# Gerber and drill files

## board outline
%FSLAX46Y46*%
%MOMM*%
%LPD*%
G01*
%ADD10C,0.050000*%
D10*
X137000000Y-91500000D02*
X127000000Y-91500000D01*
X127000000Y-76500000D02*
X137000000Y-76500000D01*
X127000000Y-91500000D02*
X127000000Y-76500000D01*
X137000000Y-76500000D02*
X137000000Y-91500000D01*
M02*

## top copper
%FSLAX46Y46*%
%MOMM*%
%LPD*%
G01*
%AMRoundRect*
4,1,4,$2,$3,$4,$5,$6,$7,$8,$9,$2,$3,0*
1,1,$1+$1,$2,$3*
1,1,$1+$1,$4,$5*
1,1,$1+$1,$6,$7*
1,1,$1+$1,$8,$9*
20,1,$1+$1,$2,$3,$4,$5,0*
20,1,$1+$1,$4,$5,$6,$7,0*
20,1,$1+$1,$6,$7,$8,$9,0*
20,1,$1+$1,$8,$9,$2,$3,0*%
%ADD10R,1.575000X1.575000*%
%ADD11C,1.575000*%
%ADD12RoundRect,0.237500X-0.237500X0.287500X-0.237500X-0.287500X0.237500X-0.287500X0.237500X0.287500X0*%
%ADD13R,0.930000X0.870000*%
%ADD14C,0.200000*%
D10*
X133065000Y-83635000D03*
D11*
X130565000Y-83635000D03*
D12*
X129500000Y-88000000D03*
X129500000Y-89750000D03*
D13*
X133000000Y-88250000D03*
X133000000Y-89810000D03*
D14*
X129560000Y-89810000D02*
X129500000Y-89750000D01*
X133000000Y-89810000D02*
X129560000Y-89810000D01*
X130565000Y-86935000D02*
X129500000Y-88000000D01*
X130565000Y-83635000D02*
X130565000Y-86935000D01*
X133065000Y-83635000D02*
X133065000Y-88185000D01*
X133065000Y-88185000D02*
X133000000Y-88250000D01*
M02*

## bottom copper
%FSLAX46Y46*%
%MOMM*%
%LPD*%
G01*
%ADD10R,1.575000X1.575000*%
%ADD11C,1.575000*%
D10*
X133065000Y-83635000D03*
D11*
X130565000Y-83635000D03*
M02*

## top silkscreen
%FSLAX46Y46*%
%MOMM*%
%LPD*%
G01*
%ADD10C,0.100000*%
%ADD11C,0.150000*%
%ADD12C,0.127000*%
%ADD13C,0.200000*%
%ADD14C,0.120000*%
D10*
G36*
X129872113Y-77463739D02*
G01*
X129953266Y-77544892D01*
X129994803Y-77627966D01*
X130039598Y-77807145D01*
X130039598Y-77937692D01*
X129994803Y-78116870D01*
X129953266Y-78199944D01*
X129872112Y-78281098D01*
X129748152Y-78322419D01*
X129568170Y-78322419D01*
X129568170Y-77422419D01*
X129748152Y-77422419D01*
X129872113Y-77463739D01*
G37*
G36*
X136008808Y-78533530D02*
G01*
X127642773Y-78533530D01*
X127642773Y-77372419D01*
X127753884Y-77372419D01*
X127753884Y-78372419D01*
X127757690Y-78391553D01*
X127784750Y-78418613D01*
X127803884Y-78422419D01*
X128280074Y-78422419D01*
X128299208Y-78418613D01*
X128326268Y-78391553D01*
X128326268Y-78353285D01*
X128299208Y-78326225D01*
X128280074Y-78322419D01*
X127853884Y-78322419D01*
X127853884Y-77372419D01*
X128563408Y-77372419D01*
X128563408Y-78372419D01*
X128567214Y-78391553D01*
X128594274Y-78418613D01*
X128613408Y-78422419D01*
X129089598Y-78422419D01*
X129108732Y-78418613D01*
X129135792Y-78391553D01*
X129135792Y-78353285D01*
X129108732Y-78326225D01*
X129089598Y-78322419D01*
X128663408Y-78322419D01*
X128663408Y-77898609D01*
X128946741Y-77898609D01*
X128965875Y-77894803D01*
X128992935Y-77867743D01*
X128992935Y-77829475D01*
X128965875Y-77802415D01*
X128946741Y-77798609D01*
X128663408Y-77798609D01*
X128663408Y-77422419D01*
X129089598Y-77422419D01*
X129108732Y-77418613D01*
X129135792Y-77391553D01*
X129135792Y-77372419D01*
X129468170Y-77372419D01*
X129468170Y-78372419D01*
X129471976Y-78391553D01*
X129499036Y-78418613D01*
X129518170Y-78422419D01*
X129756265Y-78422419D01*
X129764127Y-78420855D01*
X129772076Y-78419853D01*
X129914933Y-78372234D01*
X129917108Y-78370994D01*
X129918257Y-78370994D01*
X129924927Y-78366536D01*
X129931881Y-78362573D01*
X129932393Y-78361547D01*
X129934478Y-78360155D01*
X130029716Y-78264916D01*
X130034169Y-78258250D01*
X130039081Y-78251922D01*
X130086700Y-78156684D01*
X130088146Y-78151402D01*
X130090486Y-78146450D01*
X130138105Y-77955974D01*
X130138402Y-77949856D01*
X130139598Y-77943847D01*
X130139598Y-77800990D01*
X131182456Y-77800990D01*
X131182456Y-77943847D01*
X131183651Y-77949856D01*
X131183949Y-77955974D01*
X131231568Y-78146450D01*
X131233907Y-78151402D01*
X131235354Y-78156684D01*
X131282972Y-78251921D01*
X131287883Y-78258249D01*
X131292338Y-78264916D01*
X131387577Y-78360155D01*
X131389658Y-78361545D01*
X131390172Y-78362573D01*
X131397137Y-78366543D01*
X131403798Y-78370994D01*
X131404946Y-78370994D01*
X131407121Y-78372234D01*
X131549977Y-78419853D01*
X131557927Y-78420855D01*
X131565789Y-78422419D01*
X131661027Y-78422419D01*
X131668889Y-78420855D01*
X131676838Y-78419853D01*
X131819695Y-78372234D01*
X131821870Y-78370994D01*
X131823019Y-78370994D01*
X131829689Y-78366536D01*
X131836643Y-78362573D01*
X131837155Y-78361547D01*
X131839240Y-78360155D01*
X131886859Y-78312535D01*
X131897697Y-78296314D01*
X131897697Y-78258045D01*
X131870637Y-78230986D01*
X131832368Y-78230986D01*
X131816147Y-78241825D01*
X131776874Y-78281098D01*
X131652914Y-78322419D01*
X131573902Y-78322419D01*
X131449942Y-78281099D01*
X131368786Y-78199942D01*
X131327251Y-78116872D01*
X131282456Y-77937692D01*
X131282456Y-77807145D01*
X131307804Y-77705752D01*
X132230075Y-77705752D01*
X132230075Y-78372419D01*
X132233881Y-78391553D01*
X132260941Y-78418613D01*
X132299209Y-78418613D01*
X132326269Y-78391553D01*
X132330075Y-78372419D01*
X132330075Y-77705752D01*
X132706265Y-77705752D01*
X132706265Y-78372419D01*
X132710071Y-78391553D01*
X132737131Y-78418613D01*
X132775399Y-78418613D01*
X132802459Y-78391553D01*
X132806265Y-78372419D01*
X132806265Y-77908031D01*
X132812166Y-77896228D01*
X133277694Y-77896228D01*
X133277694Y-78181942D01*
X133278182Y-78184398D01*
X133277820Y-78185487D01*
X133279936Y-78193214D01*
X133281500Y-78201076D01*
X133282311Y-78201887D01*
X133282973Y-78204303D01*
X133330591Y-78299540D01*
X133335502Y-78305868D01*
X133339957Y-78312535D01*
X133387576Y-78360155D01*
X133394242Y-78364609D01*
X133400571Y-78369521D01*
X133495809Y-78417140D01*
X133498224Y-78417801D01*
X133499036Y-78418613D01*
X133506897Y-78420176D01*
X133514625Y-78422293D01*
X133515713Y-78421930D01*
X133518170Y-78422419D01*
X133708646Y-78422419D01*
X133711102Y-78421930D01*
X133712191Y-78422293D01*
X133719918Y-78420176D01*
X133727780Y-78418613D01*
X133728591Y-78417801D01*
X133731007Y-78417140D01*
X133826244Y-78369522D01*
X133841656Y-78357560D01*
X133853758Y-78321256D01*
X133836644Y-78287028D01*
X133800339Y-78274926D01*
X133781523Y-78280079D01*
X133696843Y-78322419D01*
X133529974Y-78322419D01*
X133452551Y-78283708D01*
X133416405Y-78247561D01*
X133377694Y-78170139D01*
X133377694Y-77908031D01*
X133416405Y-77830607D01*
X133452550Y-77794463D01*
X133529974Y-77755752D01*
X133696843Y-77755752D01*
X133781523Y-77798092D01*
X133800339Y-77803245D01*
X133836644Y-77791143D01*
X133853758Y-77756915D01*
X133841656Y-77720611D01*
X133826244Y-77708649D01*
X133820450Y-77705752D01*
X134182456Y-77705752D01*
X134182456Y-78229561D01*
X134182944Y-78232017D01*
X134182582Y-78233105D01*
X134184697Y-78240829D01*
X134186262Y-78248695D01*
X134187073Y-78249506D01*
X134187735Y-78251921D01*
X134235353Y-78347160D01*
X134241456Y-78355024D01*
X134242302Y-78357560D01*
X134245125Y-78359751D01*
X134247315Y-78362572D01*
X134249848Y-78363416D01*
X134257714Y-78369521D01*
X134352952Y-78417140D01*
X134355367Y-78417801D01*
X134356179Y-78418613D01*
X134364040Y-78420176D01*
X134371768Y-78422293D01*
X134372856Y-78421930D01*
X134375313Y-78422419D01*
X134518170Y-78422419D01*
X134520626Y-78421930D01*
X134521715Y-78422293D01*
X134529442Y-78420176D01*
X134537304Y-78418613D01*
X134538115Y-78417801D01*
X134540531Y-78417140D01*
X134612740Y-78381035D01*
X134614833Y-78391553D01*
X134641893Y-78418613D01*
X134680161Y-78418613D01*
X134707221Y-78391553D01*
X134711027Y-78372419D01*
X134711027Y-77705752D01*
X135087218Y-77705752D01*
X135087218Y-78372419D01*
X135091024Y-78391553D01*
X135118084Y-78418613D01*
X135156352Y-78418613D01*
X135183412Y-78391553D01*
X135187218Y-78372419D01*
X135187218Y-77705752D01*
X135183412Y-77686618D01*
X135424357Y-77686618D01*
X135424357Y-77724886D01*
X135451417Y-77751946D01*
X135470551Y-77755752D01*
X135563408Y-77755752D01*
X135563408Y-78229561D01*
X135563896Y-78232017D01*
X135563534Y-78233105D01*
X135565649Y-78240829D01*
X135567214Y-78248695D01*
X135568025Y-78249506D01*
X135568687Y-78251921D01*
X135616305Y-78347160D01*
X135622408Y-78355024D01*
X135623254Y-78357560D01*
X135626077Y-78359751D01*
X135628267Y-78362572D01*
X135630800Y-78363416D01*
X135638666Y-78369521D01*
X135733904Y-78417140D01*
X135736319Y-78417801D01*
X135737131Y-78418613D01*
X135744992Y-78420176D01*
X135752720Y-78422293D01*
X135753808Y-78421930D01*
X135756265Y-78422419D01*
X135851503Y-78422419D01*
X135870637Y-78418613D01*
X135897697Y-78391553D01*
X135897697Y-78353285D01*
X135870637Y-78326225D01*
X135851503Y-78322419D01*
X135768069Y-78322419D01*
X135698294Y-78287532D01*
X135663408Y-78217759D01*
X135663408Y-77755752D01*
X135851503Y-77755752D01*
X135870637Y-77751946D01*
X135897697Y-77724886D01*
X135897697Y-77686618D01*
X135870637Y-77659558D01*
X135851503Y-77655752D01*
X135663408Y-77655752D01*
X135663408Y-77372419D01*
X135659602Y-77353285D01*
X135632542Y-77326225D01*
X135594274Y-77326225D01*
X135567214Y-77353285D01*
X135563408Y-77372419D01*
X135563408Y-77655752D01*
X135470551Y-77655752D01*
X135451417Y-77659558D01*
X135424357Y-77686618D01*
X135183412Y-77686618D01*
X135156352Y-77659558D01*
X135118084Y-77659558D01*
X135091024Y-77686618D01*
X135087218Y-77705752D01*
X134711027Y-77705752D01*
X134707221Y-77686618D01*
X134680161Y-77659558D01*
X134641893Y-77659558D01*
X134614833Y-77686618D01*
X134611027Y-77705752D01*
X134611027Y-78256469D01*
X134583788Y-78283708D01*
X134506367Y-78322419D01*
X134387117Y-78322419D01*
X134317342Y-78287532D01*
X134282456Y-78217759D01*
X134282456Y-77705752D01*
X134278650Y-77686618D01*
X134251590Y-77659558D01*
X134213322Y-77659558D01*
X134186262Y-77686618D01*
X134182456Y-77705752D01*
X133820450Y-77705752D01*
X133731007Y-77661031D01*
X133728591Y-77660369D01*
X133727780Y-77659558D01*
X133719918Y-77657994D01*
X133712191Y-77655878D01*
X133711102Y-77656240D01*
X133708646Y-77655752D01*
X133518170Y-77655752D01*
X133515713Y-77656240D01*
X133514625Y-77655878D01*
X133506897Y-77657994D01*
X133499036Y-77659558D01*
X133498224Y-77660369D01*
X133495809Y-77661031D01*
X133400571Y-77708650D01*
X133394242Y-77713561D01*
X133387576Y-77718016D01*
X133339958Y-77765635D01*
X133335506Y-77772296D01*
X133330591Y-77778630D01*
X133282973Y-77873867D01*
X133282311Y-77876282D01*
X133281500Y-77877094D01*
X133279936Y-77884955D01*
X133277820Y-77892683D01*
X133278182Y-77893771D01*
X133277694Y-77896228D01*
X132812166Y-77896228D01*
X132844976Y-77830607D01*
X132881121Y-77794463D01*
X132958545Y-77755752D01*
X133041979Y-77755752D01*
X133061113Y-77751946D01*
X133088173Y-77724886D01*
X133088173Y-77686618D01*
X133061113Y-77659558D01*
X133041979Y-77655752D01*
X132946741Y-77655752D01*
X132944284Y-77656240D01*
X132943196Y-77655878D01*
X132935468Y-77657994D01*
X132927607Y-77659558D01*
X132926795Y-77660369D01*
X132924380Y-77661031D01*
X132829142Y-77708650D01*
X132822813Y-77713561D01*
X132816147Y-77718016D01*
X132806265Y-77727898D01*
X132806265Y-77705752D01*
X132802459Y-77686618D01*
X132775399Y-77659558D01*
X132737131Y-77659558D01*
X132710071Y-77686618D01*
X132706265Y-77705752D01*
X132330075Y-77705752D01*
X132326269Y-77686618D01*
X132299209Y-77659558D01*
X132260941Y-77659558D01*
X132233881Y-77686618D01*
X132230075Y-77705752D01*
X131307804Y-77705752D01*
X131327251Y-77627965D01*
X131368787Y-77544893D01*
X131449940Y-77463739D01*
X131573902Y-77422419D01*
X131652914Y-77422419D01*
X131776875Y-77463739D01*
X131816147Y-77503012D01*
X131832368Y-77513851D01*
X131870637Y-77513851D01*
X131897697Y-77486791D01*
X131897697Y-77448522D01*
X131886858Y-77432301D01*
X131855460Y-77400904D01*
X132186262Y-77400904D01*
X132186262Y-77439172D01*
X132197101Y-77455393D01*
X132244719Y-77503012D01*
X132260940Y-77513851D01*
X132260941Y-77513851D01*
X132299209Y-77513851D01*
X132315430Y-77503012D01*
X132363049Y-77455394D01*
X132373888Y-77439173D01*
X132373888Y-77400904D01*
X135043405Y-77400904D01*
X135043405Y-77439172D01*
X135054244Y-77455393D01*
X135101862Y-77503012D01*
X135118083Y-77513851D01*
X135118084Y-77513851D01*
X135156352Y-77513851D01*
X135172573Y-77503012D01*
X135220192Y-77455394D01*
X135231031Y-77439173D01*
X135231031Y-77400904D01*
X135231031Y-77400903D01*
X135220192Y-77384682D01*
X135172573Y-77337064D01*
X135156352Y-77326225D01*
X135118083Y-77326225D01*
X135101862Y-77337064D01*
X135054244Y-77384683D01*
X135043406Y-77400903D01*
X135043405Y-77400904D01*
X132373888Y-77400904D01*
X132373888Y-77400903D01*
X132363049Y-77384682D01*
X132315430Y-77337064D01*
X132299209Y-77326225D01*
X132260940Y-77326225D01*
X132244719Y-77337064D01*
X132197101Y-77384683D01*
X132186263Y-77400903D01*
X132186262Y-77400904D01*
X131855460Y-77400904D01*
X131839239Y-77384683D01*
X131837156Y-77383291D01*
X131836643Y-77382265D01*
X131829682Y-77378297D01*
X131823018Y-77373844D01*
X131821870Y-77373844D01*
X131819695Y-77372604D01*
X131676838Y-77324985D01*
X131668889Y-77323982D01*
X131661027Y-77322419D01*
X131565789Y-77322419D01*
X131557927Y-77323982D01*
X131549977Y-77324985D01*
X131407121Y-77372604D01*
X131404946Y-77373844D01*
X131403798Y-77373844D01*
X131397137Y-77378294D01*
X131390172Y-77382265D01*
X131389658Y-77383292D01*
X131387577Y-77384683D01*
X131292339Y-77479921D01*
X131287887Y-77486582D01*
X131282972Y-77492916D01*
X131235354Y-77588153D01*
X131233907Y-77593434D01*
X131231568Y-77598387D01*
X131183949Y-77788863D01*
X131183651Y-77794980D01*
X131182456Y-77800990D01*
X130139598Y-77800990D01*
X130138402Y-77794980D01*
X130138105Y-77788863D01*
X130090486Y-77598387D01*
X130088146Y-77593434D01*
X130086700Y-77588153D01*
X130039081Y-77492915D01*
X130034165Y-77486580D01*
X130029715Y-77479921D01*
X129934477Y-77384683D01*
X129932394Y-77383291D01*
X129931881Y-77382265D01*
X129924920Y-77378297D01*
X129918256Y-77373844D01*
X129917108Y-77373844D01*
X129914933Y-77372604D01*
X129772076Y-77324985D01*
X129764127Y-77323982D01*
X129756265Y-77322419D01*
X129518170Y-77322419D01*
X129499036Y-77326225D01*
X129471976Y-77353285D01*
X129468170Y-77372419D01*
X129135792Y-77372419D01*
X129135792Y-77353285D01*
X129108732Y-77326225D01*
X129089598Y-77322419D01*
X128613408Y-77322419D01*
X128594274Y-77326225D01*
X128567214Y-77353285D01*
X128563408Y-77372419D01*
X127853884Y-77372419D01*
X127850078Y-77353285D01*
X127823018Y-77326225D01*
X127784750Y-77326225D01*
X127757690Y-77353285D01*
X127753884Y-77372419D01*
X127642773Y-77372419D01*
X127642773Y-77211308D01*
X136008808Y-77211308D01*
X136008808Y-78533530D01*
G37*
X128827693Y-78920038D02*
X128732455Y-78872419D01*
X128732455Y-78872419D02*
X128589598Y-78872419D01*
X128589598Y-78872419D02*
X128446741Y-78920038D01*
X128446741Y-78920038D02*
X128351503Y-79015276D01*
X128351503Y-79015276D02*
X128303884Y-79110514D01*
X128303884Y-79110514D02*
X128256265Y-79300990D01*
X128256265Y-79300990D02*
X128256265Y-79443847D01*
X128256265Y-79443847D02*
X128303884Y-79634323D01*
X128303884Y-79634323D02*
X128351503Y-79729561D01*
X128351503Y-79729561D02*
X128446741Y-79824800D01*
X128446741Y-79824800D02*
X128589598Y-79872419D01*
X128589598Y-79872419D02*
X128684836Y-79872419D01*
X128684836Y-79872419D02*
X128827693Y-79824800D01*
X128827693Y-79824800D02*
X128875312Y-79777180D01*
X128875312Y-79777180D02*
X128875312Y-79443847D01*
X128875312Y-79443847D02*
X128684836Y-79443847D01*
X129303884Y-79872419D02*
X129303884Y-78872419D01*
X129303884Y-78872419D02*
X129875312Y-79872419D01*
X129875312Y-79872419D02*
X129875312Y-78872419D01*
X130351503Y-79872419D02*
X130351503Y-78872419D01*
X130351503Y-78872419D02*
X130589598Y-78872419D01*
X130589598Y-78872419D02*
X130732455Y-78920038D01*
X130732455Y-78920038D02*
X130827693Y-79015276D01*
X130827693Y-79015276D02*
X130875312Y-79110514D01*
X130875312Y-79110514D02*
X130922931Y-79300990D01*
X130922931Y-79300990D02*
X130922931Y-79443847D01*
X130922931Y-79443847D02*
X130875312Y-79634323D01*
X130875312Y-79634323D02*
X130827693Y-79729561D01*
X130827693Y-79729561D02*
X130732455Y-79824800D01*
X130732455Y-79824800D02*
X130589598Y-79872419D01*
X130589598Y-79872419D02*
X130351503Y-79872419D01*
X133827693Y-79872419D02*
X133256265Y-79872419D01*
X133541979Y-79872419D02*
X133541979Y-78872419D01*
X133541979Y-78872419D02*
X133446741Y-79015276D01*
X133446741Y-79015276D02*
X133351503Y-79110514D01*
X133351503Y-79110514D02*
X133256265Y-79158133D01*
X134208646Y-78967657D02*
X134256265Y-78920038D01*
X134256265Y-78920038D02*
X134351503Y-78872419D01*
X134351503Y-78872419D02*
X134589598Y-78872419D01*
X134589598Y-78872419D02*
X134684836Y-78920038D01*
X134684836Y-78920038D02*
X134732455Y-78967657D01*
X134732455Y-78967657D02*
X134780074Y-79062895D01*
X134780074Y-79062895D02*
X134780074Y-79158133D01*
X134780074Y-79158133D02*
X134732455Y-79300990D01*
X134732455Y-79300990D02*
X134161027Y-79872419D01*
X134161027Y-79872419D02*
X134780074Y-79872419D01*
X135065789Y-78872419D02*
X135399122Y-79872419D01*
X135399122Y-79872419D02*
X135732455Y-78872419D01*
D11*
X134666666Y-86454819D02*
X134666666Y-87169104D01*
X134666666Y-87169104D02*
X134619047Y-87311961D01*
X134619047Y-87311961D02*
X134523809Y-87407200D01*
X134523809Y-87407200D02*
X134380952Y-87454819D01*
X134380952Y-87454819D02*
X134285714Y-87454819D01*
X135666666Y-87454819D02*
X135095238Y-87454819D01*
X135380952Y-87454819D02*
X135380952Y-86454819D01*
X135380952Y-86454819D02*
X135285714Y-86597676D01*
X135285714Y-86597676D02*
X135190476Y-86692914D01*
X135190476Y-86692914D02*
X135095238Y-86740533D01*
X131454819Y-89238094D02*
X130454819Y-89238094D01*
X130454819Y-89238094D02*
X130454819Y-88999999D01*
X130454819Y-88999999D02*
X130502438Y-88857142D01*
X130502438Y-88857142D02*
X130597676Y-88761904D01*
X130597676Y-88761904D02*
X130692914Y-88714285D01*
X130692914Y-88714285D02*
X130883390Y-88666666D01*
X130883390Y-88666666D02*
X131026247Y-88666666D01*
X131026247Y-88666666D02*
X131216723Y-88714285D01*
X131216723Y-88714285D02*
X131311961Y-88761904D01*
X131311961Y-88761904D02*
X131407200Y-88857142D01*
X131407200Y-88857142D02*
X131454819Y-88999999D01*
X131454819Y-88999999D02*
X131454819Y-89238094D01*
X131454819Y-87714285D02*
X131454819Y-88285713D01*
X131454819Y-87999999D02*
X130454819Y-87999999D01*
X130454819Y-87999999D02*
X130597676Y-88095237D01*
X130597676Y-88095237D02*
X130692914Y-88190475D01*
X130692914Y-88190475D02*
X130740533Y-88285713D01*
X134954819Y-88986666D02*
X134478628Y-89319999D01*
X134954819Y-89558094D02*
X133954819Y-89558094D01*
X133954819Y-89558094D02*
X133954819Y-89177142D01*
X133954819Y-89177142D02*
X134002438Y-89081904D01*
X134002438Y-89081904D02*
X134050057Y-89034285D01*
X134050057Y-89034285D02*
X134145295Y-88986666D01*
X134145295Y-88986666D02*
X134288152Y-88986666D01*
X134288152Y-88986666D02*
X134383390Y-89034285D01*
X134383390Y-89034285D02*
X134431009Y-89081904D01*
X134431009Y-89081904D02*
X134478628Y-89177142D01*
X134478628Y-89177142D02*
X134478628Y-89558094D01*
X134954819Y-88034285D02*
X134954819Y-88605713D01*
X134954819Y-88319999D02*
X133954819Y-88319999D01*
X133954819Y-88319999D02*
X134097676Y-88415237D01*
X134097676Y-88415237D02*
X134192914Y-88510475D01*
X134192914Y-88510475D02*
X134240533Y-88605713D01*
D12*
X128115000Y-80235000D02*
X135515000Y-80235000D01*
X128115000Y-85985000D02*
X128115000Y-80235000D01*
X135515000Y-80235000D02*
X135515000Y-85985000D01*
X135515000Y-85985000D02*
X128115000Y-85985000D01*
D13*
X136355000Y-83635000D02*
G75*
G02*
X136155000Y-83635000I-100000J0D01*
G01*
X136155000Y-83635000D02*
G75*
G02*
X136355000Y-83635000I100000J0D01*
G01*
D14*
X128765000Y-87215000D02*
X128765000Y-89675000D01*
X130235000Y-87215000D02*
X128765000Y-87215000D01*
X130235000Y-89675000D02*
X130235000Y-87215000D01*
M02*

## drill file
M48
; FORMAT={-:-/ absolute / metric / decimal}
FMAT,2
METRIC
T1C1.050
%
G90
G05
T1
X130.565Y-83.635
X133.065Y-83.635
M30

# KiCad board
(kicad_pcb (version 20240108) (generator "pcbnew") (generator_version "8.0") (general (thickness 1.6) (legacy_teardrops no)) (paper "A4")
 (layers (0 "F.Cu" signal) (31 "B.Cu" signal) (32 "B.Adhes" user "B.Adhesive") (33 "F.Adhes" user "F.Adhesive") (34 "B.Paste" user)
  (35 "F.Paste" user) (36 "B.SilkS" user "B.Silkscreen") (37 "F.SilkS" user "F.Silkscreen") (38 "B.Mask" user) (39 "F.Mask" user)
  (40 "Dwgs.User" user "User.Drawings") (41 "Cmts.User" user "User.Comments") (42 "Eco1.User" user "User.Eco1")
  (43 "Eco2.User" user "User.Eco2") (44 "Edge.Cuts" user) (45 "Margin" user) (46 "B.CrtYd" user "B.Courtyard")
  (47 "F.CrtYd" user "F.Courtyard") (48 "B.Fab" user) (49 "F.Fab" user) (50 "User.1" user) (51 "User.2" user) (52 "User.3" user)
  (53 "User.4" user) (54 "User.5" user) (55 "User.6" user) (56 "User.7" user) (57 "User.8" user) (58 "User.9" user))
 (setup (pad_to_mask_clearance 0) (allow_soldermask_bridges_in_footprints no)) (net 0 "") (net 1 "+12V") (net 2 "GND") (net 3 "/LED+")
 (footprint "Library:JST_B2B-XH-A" (layer "F.Cu") (at 131.815 83.11)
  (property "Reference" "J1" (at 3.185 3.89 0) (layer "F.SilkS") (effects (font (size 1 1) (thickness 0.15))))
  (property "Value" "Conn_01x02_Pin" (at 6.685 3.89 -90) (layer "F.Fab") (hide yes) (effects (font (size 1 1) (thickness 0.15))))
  (fp_line (start -3.7 -2.875) (end 3.7 -2.875) (stroke (width 0.127) (type solid)) (layer "F.SilkS"))
  (fp_line (start -3.7 2.875) (end -3.7 -2.875) (stroke (width 0.127) (type solid)) (layer "F.SilkS"))
  (fp_line (start 3.7 -2.875) (end 3.7 2.875) (stroke (width 0.127) (type solid)) (layer "F.SilkS"))
  (fp_line (start 3.7 2.875) (end -3.7 2.875) (stroke (width 0.127) (type solid)) (layer "F.SilkS"))
  (fp_circle (center 4.44 0.525) (end 4.54 0.525) (stroke (width 0.2) (type solid)) (fill none) (layer "F.SilkS"))
  (pad "1" thru_hole rect (at 1.25 0.525) (size 1.575 1.575) (drill 1.05) (layers "*.Cu" "*.Mask") (remove_unused_layers no) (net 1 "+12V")
   (solder_mask_margin 0.102))
  (pad "2" thru_hole circle (at -1.25 0.525) (size 1.575 1.575) (drill 1.05) (layers "*.Cu" "*.Mask") (remove_unused_layers no)
   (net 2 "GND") (solder_mask_margin 0.102)))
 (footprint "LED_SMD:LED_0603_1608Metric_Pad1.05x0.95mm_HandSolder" (layer "F.Cu") (at 129.5 88.875 -90)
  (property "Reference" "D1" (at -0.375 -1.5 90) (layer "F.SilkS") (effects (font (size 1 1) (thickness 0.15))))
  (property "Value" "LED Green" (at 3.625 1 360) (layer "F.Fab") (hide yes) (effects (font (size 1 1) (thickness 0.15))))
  (fp_line (start -1.66 0.735) (end 0.8 0.735) (stroke (width 0.12) (type solid)) (layer "F.SilkS"))
  (fp_line (start -1.66 -0.735) (end -1.66 0.735) (stroke (width 0.12) (type solid)) (layer "F.SilkS"))
  (fp_line (start 0.8 -0.735) (end -1.66 -0.735) (stroke (width 0.12) (type solid)) (layer "F.SilkS"))
  (pad "1" smd roundrect (at -0.875 0 270) (size 1.05 0.95) (layers "F.Cu" "F.Paste" "F.Mask") (roundrect_rratio 0.25) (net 2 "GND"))
  (pad "2" smd roundrect (at 0.875 0 270) (size 1.05 0.95) (layers "F.Cu" "F.Paste" "F.Mask") (roundrect_rratio 0.25) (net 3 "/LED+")))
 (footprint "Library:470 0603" (layer "F.Cu") (at 133 89.03 -90)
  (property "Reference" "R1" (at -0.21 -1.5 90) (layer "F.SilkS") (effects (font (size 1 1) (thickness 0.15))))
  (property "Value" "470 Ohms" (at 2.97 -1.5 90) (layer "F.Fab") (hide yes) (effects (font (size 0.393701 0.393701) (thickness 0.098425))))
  (pad "1" smd rect (at -0.78 0 270) (size 0.87 0.93) (layers "F.Cu" "F.Paste" "F.Mask") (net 1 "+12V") (solder_mask_margin 0.102))
  (pad "2" smd rect (at 0.78 0 270) (size 0.87 0.93) (layers "F.Cu" "F.Paste" "F.Mask") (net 3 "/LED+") (solder_mask_margin 0.102)))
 (gr_line (start 137 91.5) (end 127 91.5) (stroke (width 0.05) (type default)) (layer "Edge.Cuts"))
 (gr_line (start 127 76.5) (end 137 76.5) (stroke (width 0.05) (type default)) (layer "Edge.Cuts"))
 (gr_line (start 127 91.5) (end 127 76.5) (stroke (width 0.05) (type default)) (layer "Edge.Cuts"))
 (gr_line (start 137 76.5) (end 137 91.5) (stroke (width 0.05) (type default)) (layer "Edge.Cuts"))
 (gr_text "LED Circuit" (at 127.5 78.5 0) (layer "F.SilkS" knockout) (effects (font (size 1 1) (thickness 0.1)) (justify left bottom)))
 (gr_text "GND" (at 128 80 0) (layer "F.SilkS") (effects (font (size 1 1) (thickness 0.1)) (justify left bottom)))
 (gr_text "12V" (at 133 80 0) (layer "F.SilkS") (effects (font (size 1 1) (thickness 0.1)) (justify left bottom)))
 (segment (start 129.56 89.81) (end 129.5 89.75) (width 0.2) (layer "F.Cu") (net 3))
 (segment (start 133 89.81) (end 129.56 89.81) (width 0.2) (layer "F.Cu") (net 3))
 (segment (start 130.565 86.935) (end 129.5 88) (width 0.2) (layer "F.Cu") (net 2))
 (segment (start 130.565 83.635) (end 130.565 86.935) (width 0.2) (layer "F.Cu") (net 2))
 (segment (start 133.065 83.635) (end 133.065 88.185) (width 0.2) (layer "F.Cu") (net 1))
 (segment (start 133.065 88.185) (end 133 88.25) (width 0.2) (layer "F.Cu") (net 1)))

